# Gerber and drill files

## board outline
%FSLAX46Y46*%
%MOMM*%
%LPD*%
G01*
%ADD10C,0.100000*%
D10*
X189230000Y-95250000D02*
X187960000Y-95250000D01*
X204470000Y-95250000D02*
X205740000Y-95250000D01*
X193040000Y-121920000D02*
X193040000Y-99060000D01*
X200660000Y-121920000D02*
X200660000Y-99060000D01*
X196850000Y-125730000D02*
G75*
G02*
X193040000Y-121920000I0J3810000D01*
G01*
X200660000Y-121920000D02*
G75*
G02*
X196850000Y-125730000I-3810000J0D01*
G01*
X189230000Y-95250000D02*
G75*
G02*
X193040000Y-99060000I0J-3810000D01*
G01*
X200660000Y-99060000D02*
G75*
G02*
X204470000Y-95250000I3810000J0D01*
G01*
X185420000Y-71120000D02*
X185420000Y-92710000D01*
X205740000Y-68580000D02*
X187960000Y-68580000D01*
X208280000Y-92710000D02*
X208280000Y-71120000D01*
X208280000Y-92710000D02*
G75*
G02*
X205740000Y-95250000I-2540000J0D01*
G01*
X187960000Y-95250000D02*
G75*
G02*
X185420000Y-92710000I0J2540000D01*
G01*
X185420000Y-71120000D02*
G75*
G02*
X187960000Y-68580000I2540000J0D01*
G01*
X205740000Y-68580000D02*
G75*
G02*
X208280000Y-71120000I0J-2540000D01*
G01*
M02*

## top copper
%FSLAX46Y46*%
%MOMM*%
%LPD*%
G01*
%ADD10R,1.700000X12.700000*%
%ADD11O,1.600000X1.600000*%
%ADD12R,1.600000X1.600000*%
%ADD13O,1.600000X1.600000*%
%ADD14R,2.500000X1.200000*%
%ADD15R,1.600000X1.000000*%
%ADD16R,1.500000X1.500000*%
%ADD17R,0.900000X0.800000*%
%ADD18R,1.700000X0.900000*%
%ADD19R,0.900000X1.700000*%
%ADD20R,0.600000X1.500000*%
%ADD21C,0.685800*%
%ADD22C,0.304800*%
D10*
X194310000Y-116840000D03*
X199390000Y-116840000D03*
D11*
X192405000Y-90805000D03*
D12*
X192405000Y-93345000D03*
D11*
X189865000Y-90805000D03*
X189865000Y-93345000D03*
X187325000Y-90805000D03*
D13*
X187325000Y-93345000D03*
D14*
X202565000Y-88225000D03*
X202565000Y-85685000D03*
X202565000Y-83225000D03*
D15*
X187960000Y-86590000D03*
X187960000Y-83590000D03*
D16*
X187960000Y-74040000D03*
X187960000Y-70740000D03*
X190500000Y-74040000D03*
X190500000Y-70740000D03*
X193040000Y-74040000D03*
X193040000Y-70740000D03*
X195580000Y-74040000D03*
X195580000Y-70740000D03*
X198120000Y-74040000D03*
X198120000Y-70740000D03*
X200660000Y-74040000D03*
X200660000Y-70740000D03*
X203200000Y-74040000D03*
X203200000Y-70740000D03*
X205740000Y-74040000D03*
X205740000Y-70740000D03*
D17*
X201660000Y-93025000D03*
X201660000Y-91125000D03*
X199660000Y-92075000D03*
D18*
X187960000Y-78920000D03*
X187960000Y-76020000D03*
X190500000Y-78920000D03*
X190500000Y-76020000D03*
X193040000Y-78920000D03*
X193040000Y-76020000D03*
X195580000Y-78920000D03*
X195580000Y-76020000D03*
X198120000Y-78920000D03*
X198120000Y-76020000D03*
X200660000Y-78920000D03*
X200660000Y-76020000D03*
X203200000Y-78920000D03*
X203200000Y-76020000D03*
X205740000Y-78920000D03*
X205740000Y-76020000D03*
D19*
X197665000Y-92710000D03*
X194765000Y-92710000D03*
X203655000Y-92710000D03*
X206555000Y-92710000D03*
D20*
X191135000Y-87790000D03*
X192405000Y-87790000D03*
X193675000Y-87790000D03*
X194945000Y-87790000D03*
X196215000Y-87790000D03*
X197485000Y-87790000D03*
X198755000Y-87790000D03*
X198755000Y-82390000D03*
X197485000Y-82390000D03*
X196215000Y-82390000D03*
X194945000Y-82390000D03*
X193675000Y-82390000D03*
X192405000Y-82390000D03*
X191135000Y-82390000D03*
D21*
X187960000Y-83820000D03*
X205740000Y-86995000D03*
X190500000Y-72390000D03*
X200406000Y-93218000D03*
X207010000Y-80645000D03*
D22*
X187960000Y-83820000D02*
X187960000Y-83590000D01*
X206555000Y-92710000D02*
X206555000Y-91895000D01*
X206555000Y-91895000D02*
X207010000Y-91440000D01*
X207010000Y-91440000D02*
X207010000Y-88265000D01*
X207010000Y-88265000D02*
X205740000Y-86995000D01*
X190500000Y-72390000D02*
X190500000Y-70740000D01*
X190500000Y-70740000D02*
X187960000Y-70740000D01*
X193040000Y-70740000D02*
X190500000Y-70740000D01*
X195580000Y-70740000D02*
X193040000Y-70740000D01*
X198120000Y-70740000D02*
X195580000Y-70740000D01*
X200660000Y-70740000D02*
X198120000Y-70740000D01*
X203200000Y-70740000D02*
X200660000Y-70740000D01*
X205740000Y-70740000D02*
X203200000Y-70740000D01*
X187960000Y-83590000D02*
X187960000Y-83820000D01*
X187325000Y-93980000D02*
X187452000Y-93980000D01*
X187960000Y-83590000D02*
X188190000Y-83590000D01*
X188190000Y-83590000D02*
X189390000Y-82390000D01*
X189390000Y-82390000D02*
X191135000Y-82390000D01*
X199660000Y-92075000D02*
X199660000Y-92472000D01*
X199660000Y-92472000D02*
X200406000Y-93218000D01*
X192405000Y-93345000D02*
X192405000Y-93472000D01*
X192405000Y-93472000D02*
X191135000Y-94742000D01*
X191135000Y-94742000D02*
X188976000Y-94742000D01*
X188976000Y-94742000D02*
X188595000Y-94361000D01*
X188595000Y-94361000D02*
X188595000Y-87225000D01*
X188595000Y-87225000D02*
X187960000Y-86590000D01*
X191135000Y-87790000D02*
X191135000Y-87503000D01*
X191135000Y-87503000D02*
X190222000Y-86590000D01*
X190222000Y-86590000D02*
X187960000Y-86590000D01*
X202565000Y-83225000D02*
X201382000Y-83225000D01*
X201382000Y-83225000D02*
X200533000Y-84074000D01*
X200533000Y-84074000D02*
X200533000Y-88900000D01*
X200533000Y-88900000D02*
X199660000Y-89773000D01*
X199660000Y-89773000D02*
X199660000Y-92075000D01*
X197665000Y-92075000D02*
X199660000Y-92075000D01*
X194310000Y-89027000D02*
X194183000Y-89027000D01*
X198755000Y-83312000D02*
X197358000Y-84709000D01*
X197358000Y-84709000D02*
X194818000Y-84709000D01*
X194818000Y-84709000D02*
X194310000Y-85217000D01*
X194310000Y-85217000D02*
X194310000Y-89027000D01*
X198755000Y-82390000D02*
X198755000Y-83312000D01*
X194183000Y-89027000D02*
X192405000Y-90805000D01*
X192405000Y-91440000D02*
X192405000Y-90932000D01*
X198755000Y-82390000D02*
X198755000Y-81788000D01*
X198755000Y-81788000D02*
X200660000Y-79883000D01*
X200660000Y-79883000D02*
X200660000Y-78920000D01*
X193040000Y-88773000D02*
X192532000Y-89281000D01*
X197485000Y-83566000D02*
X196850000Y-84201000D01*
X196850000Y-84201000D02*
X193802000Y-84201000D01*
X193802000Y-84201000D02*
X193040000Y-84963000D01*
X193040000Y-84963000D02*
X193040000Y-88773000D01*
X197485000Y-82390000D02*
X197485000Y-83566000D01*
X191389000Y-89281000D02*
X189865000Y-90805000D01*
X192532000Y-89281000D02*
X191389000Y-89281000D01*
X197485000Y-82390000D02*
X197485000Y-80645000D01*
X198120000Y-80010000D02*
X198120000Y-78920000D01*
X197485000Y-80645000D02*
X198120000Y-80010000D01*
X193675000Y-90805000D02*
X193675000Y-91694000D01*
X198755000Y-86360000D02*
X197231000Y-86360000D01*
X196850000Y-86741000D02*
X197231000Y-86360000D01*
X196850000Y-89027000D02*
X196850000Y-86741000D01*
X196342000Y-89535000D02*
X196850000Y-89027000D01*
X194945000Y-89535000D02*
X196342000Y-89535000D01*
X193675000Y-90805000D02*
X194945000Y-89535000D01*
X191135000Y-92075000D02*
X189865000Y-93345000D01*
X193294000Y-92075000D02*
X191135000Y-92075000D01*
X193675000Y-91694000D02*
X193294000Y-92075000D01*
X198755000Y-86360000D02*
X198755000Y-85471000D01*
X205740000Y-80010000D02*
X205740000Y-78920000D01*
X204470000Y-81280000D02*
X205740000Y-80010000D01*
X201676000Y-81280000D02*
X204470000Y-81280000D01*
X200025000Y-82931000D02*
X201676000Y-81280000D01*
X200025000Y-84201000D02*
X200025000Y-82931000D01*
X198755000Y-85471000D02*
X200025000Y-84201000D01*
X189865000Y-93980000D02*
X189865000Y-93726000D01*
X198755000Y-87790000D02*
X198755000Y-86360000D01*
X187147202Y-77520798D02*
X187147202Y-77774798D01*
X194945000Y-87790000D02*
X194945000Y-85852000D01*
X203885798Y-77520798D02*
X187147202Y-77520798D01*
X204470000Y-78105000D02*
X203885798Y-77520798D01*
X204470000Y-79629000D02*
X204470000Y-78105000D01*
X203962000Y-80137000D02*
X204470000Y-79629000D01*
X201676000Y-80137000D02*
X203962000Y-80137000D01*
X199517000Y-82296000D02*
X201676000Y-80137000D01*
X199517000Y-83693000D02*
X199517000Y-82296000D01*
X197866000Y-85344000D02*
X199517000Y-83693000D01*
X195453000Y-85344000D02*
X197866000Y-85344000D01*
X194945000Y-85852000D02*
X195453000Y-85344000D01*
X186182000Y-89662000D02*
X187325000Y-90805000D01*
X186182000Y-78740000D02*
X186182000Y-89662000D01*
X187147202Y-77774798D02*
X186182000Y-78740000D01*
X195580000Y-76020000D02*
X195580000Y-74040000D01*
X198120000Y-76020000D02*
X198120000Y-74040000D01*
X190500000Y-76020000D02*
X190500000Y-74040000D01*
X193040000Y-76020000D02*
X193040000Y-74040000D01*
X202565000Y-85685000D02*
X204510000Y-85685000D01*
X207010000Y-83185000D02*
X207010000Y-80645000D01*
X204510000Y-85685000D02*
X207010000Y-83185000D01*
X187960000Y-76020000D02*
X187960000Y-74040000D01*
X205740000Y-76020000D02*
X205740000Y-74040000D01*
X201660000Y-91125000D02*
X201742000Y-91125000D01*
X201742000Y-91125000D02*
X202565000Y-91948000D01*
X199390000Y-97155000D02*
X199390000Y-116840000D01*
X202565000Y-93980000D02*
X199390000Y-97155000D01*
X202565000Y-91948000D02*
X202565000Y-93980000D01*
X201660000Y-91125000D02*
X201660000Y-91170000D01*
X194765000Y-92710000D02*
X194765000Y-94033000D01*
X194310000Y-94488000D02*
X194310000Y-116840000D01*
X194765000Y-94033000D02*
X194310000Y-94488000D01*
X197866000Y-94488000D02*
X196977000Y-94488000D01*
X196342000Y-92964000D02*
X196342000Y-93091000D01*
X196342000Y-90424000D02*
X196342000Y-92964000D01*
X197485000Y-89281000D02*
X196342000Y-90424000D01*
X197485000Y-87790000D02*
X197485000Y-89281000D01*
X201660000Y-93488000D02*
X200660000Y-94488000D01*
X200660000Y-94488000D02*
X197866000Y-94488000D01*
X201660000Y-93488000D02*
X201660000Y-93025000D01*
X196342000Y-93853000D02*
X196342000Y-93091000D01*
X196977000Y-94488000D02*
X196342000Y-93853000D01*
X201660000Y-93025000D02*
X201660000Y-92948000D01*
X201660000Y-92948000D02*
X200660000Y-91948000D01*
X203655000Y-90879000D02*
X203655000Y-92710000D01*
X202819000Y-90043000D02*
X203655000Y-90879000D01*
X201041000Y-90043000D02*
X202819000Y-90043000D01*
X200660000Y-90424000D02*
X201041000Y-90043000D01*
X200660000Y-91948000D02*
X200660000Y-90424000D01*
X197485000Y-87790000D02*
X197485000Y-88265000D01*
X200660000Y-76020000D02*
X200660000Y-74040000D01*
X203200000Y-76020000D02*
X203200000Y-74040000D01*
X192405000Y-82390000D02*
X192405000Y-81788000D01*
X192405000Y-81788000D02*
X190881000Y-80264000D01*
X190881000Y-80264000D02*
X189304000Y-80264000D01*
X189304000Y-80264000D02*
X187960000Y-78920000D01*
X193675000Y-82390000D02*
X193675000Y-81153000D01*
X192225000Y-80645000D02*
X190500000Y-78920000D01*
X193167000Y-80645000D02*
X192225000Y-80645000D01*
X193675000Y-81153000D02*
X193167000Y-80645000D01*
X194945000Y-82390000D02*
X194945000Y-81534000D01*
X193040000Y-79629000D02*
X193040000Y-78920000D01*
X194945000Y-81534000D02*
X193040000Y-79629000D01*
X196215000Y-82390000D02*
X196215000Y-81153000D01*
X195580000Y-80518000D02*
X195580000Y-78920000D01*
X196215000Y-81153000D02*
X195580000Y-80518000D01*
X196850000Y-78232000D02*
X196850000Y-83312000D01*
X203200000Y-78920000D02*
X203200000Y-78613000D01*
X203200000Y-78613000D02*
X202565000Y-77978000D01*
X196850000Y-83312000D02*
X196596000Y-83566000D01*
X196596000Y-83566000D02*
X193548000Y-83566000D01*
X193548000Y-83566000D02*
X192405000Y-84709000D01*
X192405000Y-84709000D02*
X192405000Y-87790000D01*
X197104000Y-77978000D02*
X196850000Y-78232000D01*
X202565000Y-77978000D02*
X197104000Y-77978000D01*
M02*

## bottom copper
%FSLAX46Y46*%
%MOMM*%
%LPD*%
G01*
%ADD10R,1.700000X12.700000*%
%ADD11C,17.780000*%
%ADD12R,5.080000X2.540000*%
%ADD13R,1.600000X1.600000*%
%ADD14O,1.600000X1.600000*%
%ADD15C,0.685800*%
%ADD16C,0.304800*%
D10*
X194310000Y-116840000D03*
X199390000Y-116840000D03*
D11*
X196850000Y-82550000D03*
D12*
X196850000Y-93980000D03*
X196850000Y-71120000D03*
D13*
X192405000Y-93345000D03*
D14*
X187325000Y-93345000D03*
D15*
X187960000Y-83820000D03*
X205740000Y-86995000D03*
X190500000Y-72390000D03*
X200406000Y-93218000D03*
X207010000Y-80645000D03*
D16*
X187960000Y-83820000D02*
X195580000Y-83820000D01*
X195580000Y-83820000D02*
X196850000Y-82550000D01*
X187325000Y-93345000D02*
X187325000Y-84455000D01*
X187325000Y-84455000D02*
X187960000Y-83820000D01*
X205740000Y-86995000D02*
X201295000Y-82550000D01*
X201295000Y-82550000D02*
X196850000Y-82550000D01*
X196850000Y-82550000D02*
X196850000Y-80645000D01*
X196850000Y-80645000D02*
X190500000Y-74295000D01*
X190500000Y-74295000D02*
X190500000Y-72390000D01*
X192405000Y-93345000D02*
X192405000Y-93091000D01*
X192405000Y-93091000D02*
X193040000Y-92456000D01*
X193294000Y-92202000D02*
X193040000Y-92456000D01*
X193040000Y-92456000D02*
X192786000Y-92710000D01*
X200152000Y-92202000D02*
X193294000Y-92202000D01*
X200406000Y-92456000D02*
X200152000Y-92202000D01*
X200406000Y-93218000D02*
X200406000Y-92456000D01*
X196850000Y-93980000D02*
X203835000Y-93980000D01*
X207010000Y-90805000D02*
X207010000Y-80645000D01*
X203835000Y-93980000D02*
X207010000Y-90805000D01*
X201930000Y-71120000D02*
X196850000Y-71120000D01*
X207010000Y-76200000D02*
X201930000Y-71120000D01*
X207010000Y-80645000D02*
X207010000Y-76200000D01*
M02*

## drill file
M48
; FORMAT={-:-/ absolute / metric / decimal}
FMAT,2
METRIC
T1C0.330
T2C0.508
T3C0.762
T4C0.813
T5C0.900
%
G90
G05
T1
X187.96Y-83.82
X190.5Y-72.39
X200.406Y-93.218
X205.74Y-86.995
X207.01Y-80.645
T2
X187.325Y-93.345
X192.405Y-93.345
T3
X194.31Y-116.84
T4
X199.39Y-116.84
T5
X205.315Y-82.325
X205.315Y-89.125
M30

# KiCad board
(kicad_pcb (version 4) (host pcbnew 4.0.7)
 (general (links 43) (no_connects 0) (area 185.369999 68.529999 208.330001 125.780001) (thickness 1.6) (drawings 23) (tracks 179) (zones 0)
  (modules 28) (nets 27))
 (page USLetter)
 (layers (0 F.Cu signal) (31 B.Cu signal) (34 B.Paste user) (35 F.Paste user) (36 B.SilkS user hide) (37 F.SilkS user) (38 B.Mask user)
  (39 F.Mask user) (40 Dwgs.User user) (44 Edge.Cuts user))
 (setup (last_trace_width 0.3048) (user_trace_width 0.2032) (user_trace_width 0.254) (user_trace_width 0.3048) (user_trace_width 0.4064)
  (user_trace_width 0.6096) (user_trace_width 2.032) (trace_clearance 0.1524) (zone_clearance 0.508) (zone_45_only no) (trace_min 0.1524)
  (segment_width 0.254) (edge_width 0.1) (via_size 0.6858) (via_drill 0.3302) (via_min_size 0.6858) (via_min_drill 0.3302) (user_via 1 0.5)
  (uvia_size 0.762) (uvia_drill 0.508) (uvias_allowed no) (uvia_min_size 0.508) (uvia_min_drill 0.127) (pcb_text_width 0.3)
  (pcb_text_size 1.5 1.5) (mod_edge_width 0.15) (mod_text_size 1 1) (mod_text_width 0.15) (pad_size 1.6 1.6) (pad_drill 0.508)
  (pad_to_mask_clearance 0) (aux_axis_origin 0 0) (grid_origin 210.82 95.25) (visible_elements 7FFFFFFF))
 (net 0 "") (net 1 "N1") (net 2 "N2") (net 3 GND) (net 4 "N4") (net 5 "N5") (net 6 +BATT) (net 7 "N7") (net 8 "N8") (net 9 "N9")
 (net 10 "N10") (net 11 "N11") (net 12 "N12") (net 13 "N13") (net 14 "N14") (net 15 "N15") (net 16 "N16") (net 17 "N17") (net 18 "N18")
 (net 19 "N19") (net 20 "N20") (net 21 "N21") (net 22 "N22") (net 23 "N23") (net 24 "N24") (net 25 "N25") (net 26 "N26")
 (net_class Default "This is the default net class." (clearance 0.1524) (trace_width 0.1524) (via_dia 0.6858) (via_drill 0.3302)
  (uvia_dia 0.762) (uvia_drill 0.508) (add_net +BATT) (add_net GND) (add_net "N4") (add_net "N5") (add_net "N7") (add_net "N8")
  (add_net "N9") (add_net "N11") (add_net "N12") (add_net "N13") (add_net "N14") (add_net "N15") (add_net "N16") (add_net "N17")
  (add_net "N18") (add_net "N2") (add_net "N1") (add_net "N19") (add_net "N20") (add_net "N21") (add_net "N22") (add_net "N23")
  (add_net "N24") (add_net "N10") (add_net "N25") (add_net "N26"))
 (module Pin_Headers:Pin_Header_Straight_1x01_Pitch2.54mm (layer F.Cu) (at 194.31 116.84)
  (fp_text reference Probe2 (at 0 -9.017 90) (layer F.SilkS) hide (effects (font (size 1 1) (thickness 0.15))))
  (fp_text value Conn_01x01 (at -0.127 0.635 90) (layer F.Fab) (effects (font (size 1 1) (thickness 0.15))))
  (pad 1 thru_hole rect (at 0 0) (size 1.7 12.7) (drill 0.762) (layers *.Cu *.Mask) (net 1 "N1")))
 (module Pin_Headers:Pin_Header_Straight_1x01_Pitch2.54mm (layer F.Cu) (at 199.39 116.84)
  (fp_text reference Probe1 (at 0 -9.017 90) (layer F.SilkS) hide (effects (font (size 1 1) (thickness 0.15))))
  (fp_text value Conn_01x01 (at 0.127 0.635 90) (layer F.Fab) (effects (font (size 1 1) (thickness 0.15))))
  (pad 1 thru_hole rect (at 0 0) (size 1.7 12.7) (drill 0.8128) (layers *.Cu *.Mask) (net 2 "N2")))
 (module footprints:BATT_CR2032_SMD (layer B.Cu) (at 196.85 82.55 90)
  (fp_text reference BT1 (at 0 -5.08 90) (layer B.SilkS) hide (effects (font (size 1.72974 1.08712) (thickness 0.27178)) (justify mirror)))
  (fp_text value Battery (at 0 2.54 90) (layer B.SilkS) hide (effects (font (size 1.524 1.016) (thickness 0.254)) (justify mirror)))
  (pad 2 smd circle (at 0 0 90) (size 17.78 17.78) (layers B.Cu B.Paste B.Mask) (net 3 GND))
  (pad 1 smd rect (at -11.43 0 90) (size 2.54 5.08) (layers B.Cu B.Paste B.Mask) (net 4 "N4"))
  (pad 1 smd rect (at 11.43 0 90) (size 2.54 5.08) (layers B.Cu B.Paste B.Mask) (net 4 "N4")))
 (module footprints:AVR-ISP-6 (layer F.Cu) (at 192.405 90.805 270)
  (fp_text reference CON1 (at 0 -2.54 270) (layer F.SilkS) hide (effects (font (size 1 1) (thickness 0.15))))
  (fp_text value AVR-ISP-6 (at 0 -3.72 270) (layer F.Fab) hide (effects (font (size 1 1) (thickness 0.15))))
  (pad 1 smd oval (at 0 0 270) (size 1.6 1.6) (layers F.Cu F.Paste F.Mask) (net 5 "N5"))
  (pad 2 thru_hole rect (at 2.54 0 270) (size 1.6 1.6) (drill 0.508) (layers *.Cu *.Mask) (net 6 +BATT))
  (pad 3 smd oval (at 0 2.54 270) (size 1.6 1.6) (layers F.Cu F.Paste F.Mask) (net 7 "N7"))
  (pad 4 smd oval (at 2.54 2.54 270) (size 1.6 1.6) (layers F.Cu F.Paste F.Mask) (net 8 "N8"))
  (pad 5 smd oval (at 0 5.08 270) (size 1.6 1.6) (layers F.Cu F.Paste F.Mask) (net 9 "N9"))
  (pad 6 thru_hole oval (at 2.54 5.08 270) (size 1.6 1.6) (drill 0.508) (layers *.Cu *.Mask) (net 3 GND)))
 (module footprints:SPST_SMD (layer F.Cu) (at 202.565 85.725 90)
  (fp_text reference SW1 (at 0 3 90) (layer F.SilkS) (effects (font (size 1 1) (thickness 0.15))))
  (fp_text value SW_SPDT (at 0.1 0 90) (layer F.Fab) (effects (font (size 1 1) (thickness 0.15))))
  (pad "" np_thru_hole circle (at 3.4 2.75 90) (size 0.9 0.9) (drill 0.9) (layers *.Cu *.Mask))
  (pad 1 smd rect (at -2.5 0 90) (size 1.2 2.5) (layers F.Cu F.Paste F.Mask) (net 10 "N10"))
  (pad 2 smd rect (at 0.04 0 90) (size 1.2 2.5) (layers F.Cu F.Paste F.Mask) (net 4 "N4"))
  (pad 3 smd rect (at 2.5 0 90) (size 1.2 2.5) (layers F.Cu F.Paste F.Mask) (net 6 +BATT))
  (pad "" np_thru_hole circle (at -3.4 2.75 90) (size 0.9 0.9) (drill 0.9) (layers *.Cu *.Mask)))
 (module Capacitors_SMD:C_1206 (layer F.Cu) (at 187.96 85.09 90)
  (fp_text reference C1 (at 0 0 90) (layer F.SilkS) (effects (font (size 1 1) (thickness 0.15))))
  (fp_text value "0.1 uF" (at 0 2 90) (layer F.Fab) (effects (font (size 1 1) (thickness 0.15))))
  (pad 1 smd rect (at -1.5 0 90) (size 1 1.6) (layers F.Cu F.Paste F.Mask) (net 6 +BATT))
  (pad 2 smd rect (at 1.5 0 90) (size 1 1.6) (layers F.Cu F.Paste F.Mask) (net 3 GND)))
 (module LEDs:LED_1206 (layer F.Cu) (at 187.96 72.39 270)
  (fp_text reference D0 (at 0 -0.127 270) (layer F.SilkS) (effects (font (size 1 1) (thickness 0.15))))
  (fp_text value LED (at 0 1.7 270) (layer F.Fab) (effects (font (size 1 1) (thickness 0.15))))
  (pad 2 smd rect (at 1.65 0 90) (size 1.5 1.5) (layers F.Cu F.Paste F.Mask) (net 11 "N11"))
  (pad 1 smd rect (at -1.65 0 90) (size 1.5 1.5) (layers F.Cu F.Paste F.Mask) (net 3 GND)))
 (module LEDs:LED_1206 (layer F.Cu) (at 190.5 72.39 270)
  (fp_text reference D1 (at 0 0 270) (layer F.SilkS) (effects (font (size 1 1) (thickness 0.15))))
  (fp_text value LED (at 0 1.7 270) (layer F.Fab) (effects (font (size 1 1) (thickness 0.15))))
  (pad 2 smd rect (at 1.65 0 90) (size 1.5 1.5) (layers F.Cu F.Paste F.Mask) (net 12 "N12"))
  (pad 1 smd rect (at -1.65 0 90) (size 1.5 1.5) (layers F.Cu F.Paste F.Mask) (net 3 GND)))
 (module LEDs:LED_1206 (layer F.Cu) (at 193.04 72.39 270)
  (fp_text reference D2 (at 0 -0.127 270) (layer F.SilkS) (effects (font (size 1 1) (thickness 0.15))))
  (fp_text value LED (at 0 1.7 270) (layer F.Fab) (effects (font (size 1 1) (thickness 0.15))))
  (pad 2 smd rect (at 1.65 0 90) (size 1.5 1.5) (layers F.Cu F.Paste F.Mask) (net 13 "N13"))
  (pad 1 smd rect (at -1.65 0 90) (size 1.5 1.5) (layers F.Cu F.Paste F.Mask) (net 3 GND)))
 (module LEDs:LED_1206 (layer F.Cu) (at 195.58 72.39 270)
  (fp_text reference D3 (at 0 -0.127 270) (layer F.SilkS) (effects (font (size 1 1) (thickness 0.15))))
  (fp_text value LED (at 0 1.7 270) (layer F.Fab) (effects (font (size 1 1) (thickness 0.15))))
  (pad 2 smd rect (at 1.65 0 90) (size 1.5 1.5) (layers F.Cu F.Paste F.Mask) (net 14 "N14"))
  (pad 1 smd rect (at -1.65 0 90) (size 1.5 1.5) (layers F.Cu F.Paste F.Mask) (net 3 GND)))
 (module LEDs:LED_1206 (layer F.Cu) (at 198.12 72.39 270)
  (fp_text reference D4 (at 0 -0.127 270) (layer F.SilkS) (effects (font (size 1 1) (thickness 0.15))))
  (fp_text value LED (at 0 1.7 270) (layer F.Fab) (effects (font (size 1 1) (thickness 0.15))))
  (pad 2 smd rect (at 1.65 0 90) (size 1.5 1.5) (layers F.Cu F.Paste F.Mask) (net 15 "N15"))
  (pad 1 smd rect (at -1.65 0 90) (size 1.5 1.5) (layers F.Cu F.Paste F.Mask) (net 3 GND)))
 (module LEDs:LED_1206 (layer F.Cu) (at 200.66 72.39 270)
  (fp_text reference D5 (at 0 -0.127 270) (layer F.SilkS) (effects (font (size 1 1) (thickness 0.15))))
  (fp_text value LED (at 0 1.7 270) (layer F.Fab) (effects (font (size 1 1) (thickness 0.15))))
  (pad 2 smd rect (at 1.65 0 90) (size 1.5 1.5) (layers F.Cu F.Paste F.Mask) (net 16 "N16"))
  (pad 1 smd rect (at -1.65 0 90) (size 1.5 1.5) (layers F.Cu F.Paste F.Mask) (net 3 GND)))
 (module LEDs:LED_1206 (layer F.Cu) (at 203.2 72.39 270)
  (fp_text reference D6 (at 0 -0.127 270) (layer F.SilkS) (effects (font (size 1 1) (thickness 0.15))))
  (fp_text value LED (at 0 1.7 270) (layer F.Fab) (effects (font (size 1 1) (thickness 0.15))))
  (pad 2 smd rect (at 1.65 0 90) (size 1.5 1.5) (layers F.Cu F.Paste F.Mask) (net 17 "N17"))
  (pad 1 smd rect (at -1.65 0 90) (size 1.5 1.5) (layers F.Cu F.Paste F.Mask) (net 3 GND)))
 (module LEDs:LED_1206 (layer F.Cu) (at 205.74 72.39 270)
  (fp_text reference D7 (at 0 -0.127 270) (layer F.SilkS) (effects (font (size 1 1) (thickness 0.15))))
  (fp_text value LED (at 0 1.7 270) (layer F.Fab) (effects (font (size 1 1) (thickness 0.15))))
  (pad 2 smd rect (at 1.65 0 90) (size 1.5 1.5) (layers F.Cu F.Paste F.Mask) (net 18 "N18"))
  (pad 1 smd rect (at -1.65 0 90) (size 1.5 1.5) (layers F.Cu F.Paste F.Mask) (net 3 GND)))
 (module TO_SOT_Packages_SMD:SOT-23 (layer F.Cu) (at 200.66 92.075 180)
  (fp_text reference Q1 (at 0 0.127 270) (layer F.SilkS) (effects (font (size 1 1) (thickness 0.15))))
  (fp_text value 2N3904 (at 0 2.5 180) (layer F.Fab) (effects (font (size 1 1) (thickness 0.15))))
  (pad 1 smd rect (at -1 -0.95 180) (size 0.9 0.8) (layers F.Cu F.Paste F.Mask) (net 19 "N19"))
  (pad 2 smd rect (at -1 0.95 180) (size 0.9 0.8) (layers F.Cu F.Paste F.Mask) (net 2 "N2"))
  (pad 3 smd rect (at 1 0 180) (size 0.9 0.8) (layers F.Cu F.Paste F.Mask) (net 6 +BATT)))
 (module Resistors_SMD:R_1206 (layer F.Cu) (at 187.96 77.47 90)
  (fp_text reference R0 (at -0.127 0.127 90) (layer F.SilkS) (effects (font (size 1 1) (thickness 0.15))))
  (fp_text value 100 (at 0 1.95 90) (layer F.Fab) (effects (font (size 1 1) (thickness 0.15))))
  (pad 1 smd rect (at -1.45 0 90) (size 0.9 1.7) (layers F.Cu F.Paste F.Mask) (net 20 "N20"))
  (pad 2 smd rect (at 1.45 0 90) (size 0.9 1.7) (layers F.Cu F.Paste F.Mask) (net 11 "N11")))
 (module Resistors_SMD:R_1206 (layer F.Cu) (at 190.5 77.47 90)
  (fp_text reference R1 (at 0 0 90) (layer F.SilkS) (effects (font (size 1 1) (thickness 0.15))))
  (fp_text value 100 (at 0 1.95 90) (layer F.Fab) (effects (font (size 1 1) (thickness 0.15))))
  (pad 1 smd rect (at -1.45 0 90) (size 0.9 1.7) (layers F.Cu F.Paste F.Mask) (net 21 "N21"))
  (pad 2 smd rect (at 1.45 0 90) (size 0.9 1.7) (layers F.Cu F.Paste F.Mask) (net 12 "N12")))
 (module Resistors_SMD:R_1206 (layer F.Cu) (at 193.04 77.47 90)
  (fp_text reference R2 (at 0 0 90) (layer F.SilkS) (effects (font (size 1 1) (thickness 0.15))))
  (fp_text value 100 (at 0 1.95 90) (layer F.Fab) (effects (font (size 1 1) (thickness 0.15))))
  (pad 1 smd rect (at -1.45 0 90) (size 0.9 1.7) (layers F.Cu F.Paste F.Mask) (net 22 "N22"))
  (pad 2 smd rect (at 1.45 0 90) (size 0.9 1.7) (layers F.Cu F.Paste F.Mask) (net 13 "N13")))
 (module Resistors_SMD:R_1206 (layer F.Cu) (at 195.58 77.47 90)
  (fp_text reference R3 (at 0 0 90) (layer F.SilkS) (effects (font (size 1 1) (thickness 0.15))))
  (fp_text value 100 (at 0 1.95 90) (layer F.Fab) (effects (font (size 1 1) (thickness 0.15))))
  (pad 1 smd rect (at -1.45 0 90) (size 0.9 1.7) (layers F.Cu F.Paste F.Mask) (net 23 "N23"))
  (pad 2 smd rect (at 1.45 0 90) (size 0.9 1.7) (layers F.Cu F.Paste F.Mask) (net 14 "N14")))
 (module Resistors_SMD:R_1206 (layer F.Cu) (at 198.12 77.47 90)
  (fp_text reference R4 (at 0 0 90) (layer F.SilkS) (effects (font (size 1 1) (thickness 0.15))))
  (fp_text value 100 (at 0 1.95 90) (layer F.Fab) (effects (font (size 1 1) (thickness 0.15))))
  (pad 1 smd rect (at -1.45 0 90) (size 0.9 1.7) (layers F.Cu F.Paste F.Mask) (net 7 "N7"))
  (pad 2 smd rect (at 1.45 0 90) (size 0.9 1.7) (layers F.Cu F.Paste F.Mask) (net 15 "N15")))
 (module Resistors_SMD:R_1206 (layer F.Cu) (at 200.66 77.47 90)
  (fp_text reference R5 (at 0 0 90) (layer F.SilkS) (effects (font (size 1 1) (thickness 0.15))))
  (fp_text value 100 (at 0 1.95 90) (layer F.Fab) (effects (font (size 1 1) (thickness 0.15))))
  (pad 1 smd rect (at -1.45 0 90) (size 0.9 1.7) (layers F.Cu F.Paste F.Mask) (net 5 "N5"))
  (pad 2 smd rect (at 1.45 0 90) (size 0.9 1.7) (layers F.Cu F.Paste F.Mask) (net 16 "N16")))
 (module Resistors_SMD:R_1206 (layer F.Cu) (at 203.2 77.47 90)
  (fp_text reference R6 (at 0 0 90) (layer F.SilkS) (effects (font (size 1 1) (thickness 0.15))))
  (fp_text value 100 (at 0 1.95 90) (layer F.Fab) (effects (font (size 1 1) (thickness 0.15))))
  (pad 1 smd rect (at -1.45 0 90) (size 0.9 1.7) (layers F.Cu F.Paste F.Mask) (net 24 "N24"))
  (pad 2 smd rect (at 1.45 0 90) (size 0.9 1.7) (layers F.Cu F.Paste F.Mask) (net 17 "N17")))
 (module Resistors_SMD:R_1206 (layer F.Cu) (at 205.74 77.47 90)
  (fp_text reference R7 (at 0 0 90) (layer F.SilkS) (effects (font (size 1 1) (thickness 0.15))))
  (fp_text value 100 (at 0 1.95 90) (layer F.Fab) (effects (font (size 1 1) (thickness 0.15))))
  (pad 1 smd rect (at -1.45 0 90) (size 0.9 1.7) (layers F.Cu F.Paste F.Mask) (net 8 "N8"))
  (pad 2 smd rect (at 1.45 0 90) (size 0.9 1.7) (layers F.Cu F.Paste F.Mask) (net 18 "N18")))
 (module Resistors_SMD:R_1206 (layer F.Cu) (at 196.215 92.71 180)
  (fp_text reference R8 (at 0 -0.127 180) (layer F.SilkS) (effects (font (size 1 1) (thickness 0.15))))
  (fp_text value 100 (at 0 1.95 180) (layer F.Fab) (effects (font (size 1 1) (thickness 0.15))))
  (pad 1 smd rect (at -1.45 0 180) (size 0.9 1.7) (layers F.Cu F.Paste F.Mask) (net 6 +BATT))
  (pad 2 smd rect (at 1.45 0 180) (size 0.9 1.7) (layers F.Cu F.Paste F.Mask) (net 1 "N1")))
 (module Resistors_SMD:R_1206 (layer F.Cu) (at 205.105 92.71)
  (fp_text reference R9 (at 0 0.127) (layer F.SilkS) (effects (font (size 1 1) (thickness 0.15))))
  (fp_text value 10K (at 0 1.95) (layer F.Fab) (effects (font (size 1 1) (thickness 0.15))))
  (pad 1 smd rect (at -1.45 0) (size 0.9 1.7) (layers F.Cu F.Paste F.Mask) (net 19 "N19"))
  (pad 2 smd rect (at 1.45 0) (size 0.9 1.7) (layers F.Cu F.Paste F.Mask) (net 3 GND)))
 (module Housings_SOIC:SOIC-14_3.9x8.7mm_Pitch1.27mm (layer F.Cu) (at 194.945 85.09 90)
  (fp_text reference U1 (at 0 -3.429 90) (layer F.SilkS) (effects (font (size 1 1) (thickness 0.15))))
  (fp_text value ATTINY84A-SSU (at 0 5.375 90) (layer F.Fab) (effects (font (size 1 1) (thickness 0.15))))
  (pad 1 smd rect (at -2.7 -3.81 90) (size 1.5 0.6) (layers F.Cu F.Paste F.Mask) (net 6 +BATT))
  (pad 2 smd rect (at -2.7 -2.54 90) (size 1.5 0.6) (layers F.Cu F.Paste F.Mask) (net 24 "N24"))
  (pad 3 smd rect (at -2.7 -1.27 90) (size 1.5 0.6) (layers F.Cu F.Paste F.Mask) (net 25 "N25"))
  (pad 4 smd rect (at -2.7 0 90) (size 1.5 0.6) (layers F.Cu F.Paste F.Mask) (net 9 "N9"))
  (pad 5 smd rect (at -2.7 1.27 90) (size 1.5 0.6) (layers F.Cu F.Paste F.Mask) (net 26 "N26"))
  (pad 6 smd rect (at -2.7 2.54 90) (size 1.5 0.6) (layers F.Cu F.Paste F.Mask) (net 19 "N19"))
  (pad 7 smd rect (at -2.7 3.81 90) (size 1.5 0.6) (layers F.Cu F.Paste F.Mask) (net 8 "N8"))
  (pad 8 smd rect (at 2.7 3.81 90) (size 1.5 0.6) (layers F.Cu F.Paste F.Mask) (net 5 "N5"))
  (pad 9 smd rect (at 2.7 2.54 90) (size 1.5 0.6) (layers F.Cu F.Paste F.Mask) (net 7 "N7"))
  (pad 10 smd rect (at 2.7 1.27 90) (size 1.5 0.6) (layers F.Cu F.Paste F.Mask) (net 23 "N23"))
  (pad 11 smd rect (at 2.7 0 90) (size 1.5 0.6) (layers F.Cu F.Paste F.Mask) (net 22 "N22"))
  (pad 12 smd rect (at 2.7 -1.27 90) (size 1.5 0.6) (layers F.Cu F.Paste F.Mask) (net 21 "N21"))
  (pad 13 smd rect (at 2.7 -2.54 90) (size 1.5 0.6) (layers F.Cu F.Paste F.Mask) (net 20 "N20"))
  (pad 14 smd rect (at 2.7 -3.81 90) (size 1.5 0.6) (layers F.Cu F.Paste F.Mask) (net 3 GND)))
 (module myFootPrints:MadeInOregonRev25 (layer F.Cu) (at 196.977 99.695 270)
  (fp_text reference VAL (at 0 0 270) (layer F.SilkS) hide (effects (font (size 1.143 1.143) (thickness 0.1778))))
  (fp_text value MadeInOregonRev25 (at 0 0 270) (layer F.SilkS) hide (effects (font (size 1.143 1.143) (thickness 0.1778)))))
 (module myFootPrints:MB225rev (layer F.Cu) (at 196.85 106.68 270)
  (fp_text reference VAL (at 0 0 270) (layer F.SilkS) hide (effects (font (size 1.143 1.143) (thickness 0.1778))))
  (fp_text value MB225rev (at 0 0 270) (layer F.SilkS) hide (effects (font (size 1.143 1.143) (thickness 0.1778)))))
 (gr_line (start 189.23 95.25) (end 187.96 95.25) (angle 90) (layer Edge.Cuts) (width 0.1))
 (gr_line (start 204.47 95.25) (end 205.74 95.25) (angle 90) (layer Edge.Cuts) (width 0.1))
 (gr_line (start 193.04 121.92) (end 193.04 99.06) (angle 90) (layer Edge.Cuts) (width 0.1))
 (gr_line (start 200.66 121.92) (end 200.66 99.06) (angle 90) (layer Edge.Cuts) (width 0.1))
 (gr_arc (start 196.85 121.92) (end 196.85 125.73) (angle 90) (layer Edge.Cuts) (width 0.1))
 (gr_arc (start 196.85 121.92) (end 200.66 121.92) (angle 90) (layer Edge.Cuts) (width 0.1))
 (gr_arc (start 189.23 99.06) (end 189.23 95.25) (angle 90) (layer Edge.Cuts) (width 0.1))
 (gr_arc (start 204.47 99.06) (end 200.66 99.06) (angle 90) (layer Edge.Cuts) (width 0.1))
 (gr_line (start 185.42 71.12) (end 185.42 92.71) (angle 90) (layer Edge.Cuts) (width 0.1))
 (gr_line (start 205.74 68.58) (end 187.96 68.58) (angle 90) (layer Edge.Cuts) (width 0.1))
 (gr_line (start 208.28 92.71) (end 208.28 71.12) (angle 90) (layer Edge.Cuts) (width 0.1))
 (gr_arc (start 205.74 92.71) (end 208.28 92.71) (angle 90) (layer Edge.Cuts) (width 0.1))
 (gr_arc (start 187.96 92.71) (end 187.96 95.25) (angle 90) (layer Edge.Cuts) (width 0.1))
 (gr_arc (start 187.96 71.12) (end 185.42 71.12) (angle 90) (layer Edge.Cuts) (width 0.1))
 (gr_arc (start 205.74 71.12) (end 205.74 68.58) (angle 90) (layer Edge.Cuts) (width 0.1))
 (segment (start 187.96 83.82) (end 195.58 83.82) (width 0.3048) (layer B.Cu) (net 3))
 (segment (start 195.58 83.82) (end 196.85 82.55) (width 0.3048) (layer B.Cu) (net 3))
 (segment (start 187.325 93.345) (end 187.325 84.455) (width 0.3048) (layer B.Cu) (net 3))
 (via (at 187.96 83.82) (size 0.6858) (drill 0.3302) (layers F.Cu B.Cu) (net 3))
 (segment (start 187.325 84.455) (end 187.96 83.82) (width 0.3048) (layer B.Cu) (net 3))
 (segment (start 187.96 83.82) (end 187.96 83.59) (width 0.3048) (layer F.Cu) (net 3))
 (segment (start 206.555 92.71) (end 206.555 91.895) (width 0.3048) (layer F.Cu) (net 3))
 (segment (start 206.555 91.895) (end 207.01 91.44) (width 0.3048) (layer F.Cu) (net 3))
 (segment (start 207.01 91.44) (end 207.01 88.265) (width 0.3048) (layer F.Cu) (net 3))
 (segment (start 207.01 88.265) (end 205.74 86.995) (width 0.3048) (layer F.Cu) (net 3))
 (via (at 205.74 86.995) (size 0.6858) (drill 0.3302) (layers F.Cu B.Cu) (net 3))
 (segment (start 205.74 86.995) (end 201.295 82.55) (width 0.3048) (layer B.Cu) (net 3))
 (segment (start 201.295 82.55) (end 196.85 82.55) (width 0.3048) (layer B.Cu) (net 3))
 (segment (start 196.85 82.55) (end 196.85 80.645) (width 0.3048) (layer B.Cu) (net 3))
 (segment (start 196.85 80.645) (end 190.5 74.295) (width 0.3048) (layer B.Cu) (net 3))
 (segment (start 190.5 74.295) (end 190.5 72.39) (width 0.3048) (layer B.Cu) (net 3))
 (via (at 190.5 72.39) (size 0.6858) (drill 0.3302) (layers F.Cu B.Cu) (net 3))
 (segment (start 190.5 72.39) (end 190.5 70.74) (width 0.3048) (layer F.Cu) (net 3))
 (segment (start 190.5 70.74) (end 187.96 70.74) (width 0.3048) (layer F.Cu) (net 3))
 (segment (start 193.04 70.74) (end 190.5 70.74) (width 0.3048) (layer F.Cu) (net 3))
 (segment (start 195.58 70.74) (end 193.04 70.74) (width 0.3048) (layer F.Cu) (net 3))
 (segment (start 198.12 70.74) (end 195.58 70.74) (width 0.3048) (layer F.Cu) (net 3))
 (segment (start 200.66 70.74) (end 198.12 70.74) (width 0.3048) (layer F.Cu) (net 3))
 (segment (start 203.2 70.74) (end 200.66 70.74) (width 0.3048) (layer F.Cu) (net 3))
 (segment (start 205.74 70.74) (end 203.2 70.74) (width 0.3048) (layer F.Cu) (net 3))
 (segment (start 187.96 83.59) (end 187.96 83.82) (width 0.3048) (layer F.Cu) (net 3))
 (segment (start 187.325 93.98) (end 187.452 93.98) (width 0.3048) (layer F.Cu) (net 3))
 (segment (start 187.96 83.59) (end 188.19 83.59) (width 0.3048) (layer F.Cu) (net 3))
 (segment (start 188.19 83.59) (end 189.39 82.39) (width 0.3048) (layer F.Cu) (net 3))
 (segment (start 189.39 82.39) (end 191.135 82.39) (width 0.3048) (layer F.Cu) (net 3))
 (segment (start 192.405 93.345) (end 192.405 93.091) (width 0.3048) (layer B.Cu) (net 6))
 (segment (start 192.405 93.091) (end 193.04 92.456) (width 0.3048) (layer B.Cu) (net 6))
 (segment (start 199.66 92.075) (end 199.66 92.472) (width 0.3048) (layer F.Cu) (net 6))
 (segment (start 199.66 92.472) (end 200.406 93.218) (width 0.3048) (layer F.Cu) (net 6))
 (segment (start 193.294 92.202) (end 193.04 92.456) (width 0.3048) (layer B.Cu) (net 6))
 (segment (start 193.04 92.456) (end 192.786 92.71) (width 0.3048) (layer B.Cu) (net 6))
 (segment (start 200.152 92.202) (end 193.294 92.202) (width 0.3048) (layer B.Cu) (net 6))
 (segment (start 200.406 92.456) (end 200.152 92.202) (width 0.3048) (layer B.Cu) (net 6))
 (segment (start 200.406 93.218) (end 200.406 92.456) (width 0.3048) (layer B.Cu) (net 6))
 (via (at 200.406 93.218) (size 0.6858) (drill 0.3302) (layers F.Cu B.Cu) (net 6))
 (segment (start 192.405 93.345) (end 192.405 93.472) (width 0.3048) (layer F.Cu) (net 6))
 (segment (start 192.405 93.472) (end 191.135 94.742) (width 0.3048) (layer F.Cu) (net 6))
 (segment (start 191.135 94.742) (end 188.976 94.742) (width 0.3048) (layer F.Cu) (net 6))
 (segment (start 188.976 94.742) (end 188.595 94.361) (width 0.3048) (layer F.Cu) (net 6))
 (segment (start 188.595 94.361) (end 188.595 87.225) (width 0.3048) (layer F.Cu) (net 6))
 (segment (start 188.595 87.225) (end 187.96 86.59) (width 0.3048) (layer F.Cu) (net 6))
 (segment (start 191.135 87.79) (end 191.135 87.503) (width 0.3048) (layer F.Cu) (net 6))
 (segment (start 191.135 87.503) (end 190.222 86.59) (width 0.3048) (layer F.Cu) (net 6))
 (segment (start 190.222 86.59) (end 187.96 86.59) (width 0.3048) (layer F.Cu) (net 6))
 (segment (start 202.565 83.225) (end 201.382 83.225) (width 0.3048) (layer F.Cu) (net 6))
 (segment (start 201.382 83.225) (end 200.533 84.074) (width 0.3048) (layer F.Cu) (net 6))
 (segment (start 200.533 84.074) (end 200.533 88.9) (width 0.3048) (layer F.Cu) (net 6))
 (segment (start 200.533 88.9) (end 199.66 89.773) (width 0.3048) (layer F.Cu) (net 6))
 (segment (start 199.66 89.773) (end 199.66 92.075) (width 0.3048) (layer F.Cu) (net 6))
 (segment (start 197.665 92.075) (end 199.66 92.075) (width 0.3048) (layer F.Cu) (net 6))
 (segment (start 194.31 89.027) (end 194.183 89.027) (width 0.3048) (layer F.Cu) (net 5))
 (segment (start 198.755 83.312) (end 197.358 84.709) (width 0.3048) (layer F.Cu) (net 5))
 (segment (start 197.358 84.709) (end 194.818 84.709) (width 0.3048) (layer F.Cu) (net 5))
 (segment (start 194.818 84.709) (end 194.31 85.217) (width 0.3048) (layer F.Cu) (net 5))
 (segment (start 194.31 85.217) (end 194.31 89.027) (width 0.3048) (layer F.Cu) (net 5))
 (segment (start 198.755 82.39) (end 198.755 83.312) (width 0.3048) (layer F.Cu) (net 5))
 (segment (start 194.183 89.027) (end 192.405 90.805) (width 0.3048) (layer F.Cu) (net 5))
 (segment (start 192.405 91.44) (end 192.405 90.932) (width 0.3048) (layer F.Cu) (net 5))
 (segment (start 198.755 82.39) (end 198.755 81.788) (width 0.3048) (layer F.Cu) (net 5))
 (segment (start 198.755 81.788) (end 200.66 79.883) (width 0.3048) (layer F.Cu) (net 5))
 (segment (start 200.66 79.883) (end 200.66 78.92) (width 0.3048) (layer F.Cu) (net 5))
 (segment (start 193.04 88.773) (end 192.532 89.281) (width 0.3048) (layer F.Cu) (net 7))
 (segment (start 197.485 83.566) (end 196.85 84.201) (width 0.3048) (layer F.Cu) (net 7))
 (segment (start 196.85 84.201) (end 193.802 84.201) (width 0.3048) (layer F.Cu) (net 7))
 (segment (start 193.802 84.201) (end 193.04 84.963) (width 0.3048) (layer F.Cu) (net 7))
 (segment (start 193.04 84.963) (end 193.04 88.773) (width 0.3048) (layer F.Cu) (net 7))
 (segment (start 197.485 82.39) (end 197.485 83.566) (width 0.3048) (layer F.Cu) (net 7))
 (segment (start 191.389 89.281) (end 189.865 90.805) (width 0.3048) (layer F.Cu) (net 7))
 (segment (start 192.532 89.281) (end 191.389 89.281) (width 0.3048) (layer F.Cu) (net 7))
 (segment (start 197.485 82.39) (end 197.485 80.645) (width 0.3048) (layer F.Cu) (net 7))
 (segment (start 198.12 80.01) (end 198.12 78.92) (width 0.3048) (layer F.Cu) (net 7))
 (segment (start 197.485 80.645) (end 198.12 80.01) (width 0.3048) (layer F.Cu) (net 7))
 (segment (start 193.675 90.805) (end 193.675 91.694) (width 0.3048) (layer F.Cu) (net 8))
 (segment (start 198.755 86.36) (end 197.231 86.36) (width 0.3048) (layer F.Cu) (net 8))
 (segment (start 196.85 86.741) (end 197.231 86.36) (width 0.3048) (layer F.Cu) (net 8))
 (segment (start 196.85 89.027) (end 196.85 86.741) (width 0.3048) (layer F.Cu) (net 8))
 (segment (start 196.342 89.535) (end 196.85 89.027) (width 0.3048) (layer F.Cu) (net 8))
 (segment (start 194.945 89.535) (end 196.342 89.535) (width 0.3048) (layer F.Cu) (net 8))
 (segment (start 193.675 90.805) (end 194.945 89.535) (width 0.3048) (layer F.Cu) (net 8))
 (segment (start 191.135 92.075) (end 189.865 93.345) (width 0.3048) (layer F.Cu) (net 8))
 (segment (start 193.294 92.075) (end 191.135 92.075) (width 0.3048) (layer F.Cu) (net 8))
 (segment (start 193.675 91.694) (end 193.294 92.075) (width 0.3048) (layer F.Cu) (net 8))
 (segment (start 198.755 86.36) (end 198.755 85.471) (width 0.3048) (layer F.Cu) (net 8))
 (segment (start 205.74 80.01) (end 205.74 78.92) (width 0.3048) (layer F.Cu) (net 8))
 (segment (start 204.47 81.28) (end 205.74 80.01) (width 0.3048) (layer F.Cu) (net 8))
 (segment (start 201.676 81.28) (end 204.47 81.28) (width 0.3048) (layer F.Cu) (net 8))
 (segment (start 200.025 82.931) (end 201.676 81.28) (width 0.3048) (layer F.Cu) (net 8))
 (segment (start 200.025 84.201) (end 200.025 82.931) (width 0.3048) (layer F.Cu) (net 8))
 (segment (start 198.755 85.471) (end 200.025 84.201) (width 0.3048) (layer F.Cu) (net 8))
 (segment (start 189.865 93.98) (end 189.865 93.726) (width 0.3048) (layer F.Cu) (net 8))
 (segment (start 198.755 87.79) (end 198.755 86.36) (width 0.3048) (layer F.Cu) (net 8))
 (segment (start 187.147202 77.520798) (end 187.147202 77.774798) (width 0.3048) (layer F.Cu) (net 9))
 (segment (start 194.945 87.79) (end 194.945 85.852) (width 0.3048) (layer F.Cu) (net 9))
 (segment (start 203.885798 77.520798) (end 187.147202 77.520798) (width 0.3048) (layer F.Cu) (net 9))
 (segment (start 204.47 78.105) (end 203.885798 77.520798) (width 0.3048) (layer F.Cu) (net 9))
 (segment (start 204.47 79.629) (end 204.47 78.105) (width 0.3048) (layer F.Cu) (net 9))
 (segment (start 203.962 80.137) (end 204.47 79.629) (width 0.3048) (layer F.Cu) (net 9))
 (segment (start 201.676 80.137) (end 203.962 80.137) (width 0.3048) (layer F.Cu) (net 9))
 (segment (start 199.517 82.296) (end 201.676 80.137) (width 0.3048) (layer F.Cu) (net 9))
 (segment (start 199.517 83.693) (end 199.517 82.296) (width 0.3048) (layer F.Cu) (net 9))
 (segment (start 197.866 85.344) (end 199.517 83.693) (width 0.3048) (layer F.Cu) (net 9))
 (segment (start 195.453 85.344) (end 197.866 85.344) (width 0.3048) (layer F.Cu) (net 9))
 (segment (start 194.945 85.852) (end 195.453 85.344) (width 0.3048) (layer F.Cu) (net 9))
 (segment (start 186.182 89.662) (end 187.325 90.805) (width 0.3048) (layer F.Cu) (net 9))
 (segment (start 186.182 78.74) (end 186.182 89.662) (width 0.3048) (layer F.Cu) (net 9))
 (segment (start 187.147202 77.774798) (end 186.182 78.74) (width 0.3048) (layer F.Cu) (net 9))
 (segment (start 195.58 76.02) (end 195.58 74.04) (width 0.3048) (layer F.Cu) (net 14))
 (segment (start 198.12 76.02) (end 198.12 74.04) (width 0.3048) (layer F.Cu) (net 15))
 (segment (start 190.5 76.02) (end 190.5 74.04) (width 0.3048) (layer F.Cu) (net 12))
 (segment (start 193.04 76.02) (end 193.04 74.04) (width 0.3048) (layer F.Cu) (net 13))
 (segment (start 196.85 93.98) (end 203.835 93.98) (width 0.3048) (layer B.Cu) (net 4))
 (segment (start 207.01 90.805) (end 207.01 80.645) (width 0.3048) (layer B.Cu) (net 4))
 (segment (start 203.835 93.98) (end 207.01 90.805) (width 0.3048) (layer B.Cu) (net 4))
 (segment (start 202.565 85.685) (end 204.51 85.685) (width 0.3048) (layer F.Cu) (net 4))
 (segment (start 201.93 71.12) (end 196.85 71.12) (width 0.3048) (layer B.Cu) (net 4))
 (segment (start 207.01 76.2) (end 201.93 71.12) (width 0.3048) (layer B.Cu) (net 4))
 (segment (start 207.01 80.645) (end 207.01 76.2) (width 0.3048) (layer B.Cu) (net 4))
 (via (at 207.01 80.645) (size 0.6858) (drill 0.3302) (layers F.Cu B.Cu) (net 4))
 (segment (start 207.01 83.185) (end 207.01 80.645) (width 0.3048) (layer F.Cu) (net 4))
 (segment (start 204.51 85.685) (end 207.01 83.185) (width 0.3048) (layer F.Cu) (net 4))
 (segment (start 187.96 76.02) (end 187.96 74.04) (width 0.3048) (layer F.Cu) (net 11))
 (segment (start 205.74 76.02) (end 205.74 74.04) (width 0.3048) (layer F.Cu) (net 18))
 (segment (start 201.66 91.125) (end 201.742 91.125) (width 0.3048) (layer F.Cu) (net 2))
 (segment (start 201.742 91.125) (end 202.565 91.948) (width 0.3048) (layer F.Cu) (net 2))
 (segment (start 199.39 97.155) (end 199.39 116.84) (width 0.3048) (layer F.Cu) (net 2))
 (segment (start 202.565 93.98) (end 199.39 97.155) (width 0.3048) (layer F.Cu) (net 2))
 (segment (start 202.565 91.948) (end 202.565 93.98) (width 0.3048) (layer F.Cu) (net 2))
 (segment (start 201.66 91.125) (end 201.66 91.17) (width 0.3048) (layer F.Cu) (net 2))
 (segment (start 194.765 92.71) (end 194.765 94.033) (width 0.3048) (layer F.Cu) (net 1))
 (segment (start 194.31 94.488) (end 194.31 116.84) (width 0.3048) (layer F.Cu) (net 1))
 (segment (start 194.765 94.033) (end 194.31 94.488) (width 0.3048) (layer F.Cu) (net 1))
 (segment (start 197.866 94.488) (end 196.977 94.488) (width 0.3048) (layer F.Cu) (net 19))
 (segment (start 196.342 92.964) (end 196.342 93.091) (width 0.3048) (layer F.Cu) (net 19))
 (segment (start 196.342 90.424) (end 196.342 92.964) (width 0.3048) (layer F.Cu) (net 19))
 (segment (start 197.485 89.281) (end 196.342 90.424) (width 0.3048) (layer F.Cu) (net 19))
 (segment (start 197.485 87.79) (end 197.485 89.281) (width 0.3048) (layer F.Cu) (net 19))
 (segment (start 201.66 93.488) (end 200.66 94.488) (width 0.3048) (layer F.Cu) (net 19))
 (segment (start 200.66 94.488) (end 197.866 94.488) (width 0.3048) (layer F.Cu) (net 19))
 (segment (start 201.66 93.488) (end 201.66 93.025) (width 0.3048) (layer F.Cu) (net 19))
 (segment (start 196.342 93.853) (end 196.342 93.091) (width 0.3048) (layer F.Cu) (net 19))
 (segment (start 196.977 94.488) (end 196.342 93.853) (width 0.3048) (layer F.Cu) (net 19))
 (segment (start 201.66 93.025) (end 201.66 92.948) (width 0.3048) (layer F.Cu) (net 19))
 (segment (start 201.66 92.948) (end 200.66 91.948) (width 0.3048) (layer F.Cu) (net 19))
 (segment (start 203.655 90.879) (end 203.655 92.71) (width 0.3048) (layer F.Cu) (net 19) (status 20))
 (segment (start 202.819 90.043) (end 203.655 90.879) (width 0.3048) (layer F.Cu) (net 19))
 (segment (start 201.041 90.043) (end 202.819 90.043) (width 0.3048) (layer F.Cu) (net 19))
 (segment (start 200.66 90.424) (end 201.041 90.043) (width 0.3048) (layer F.Cu) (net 19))
 (segment (start 200.66 91.948) (end 200.66 90.424) (width 0.3048) (layer F.Cu) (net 19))
 (segment (start 197.485 87.79) (end 197.485 88.265) (width 0.3048) (layer F.Cu) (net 19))
 (segment (start 200.66 76.02) (end 200.66 74.04) (width 0.3048) (layer F.Cu) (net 16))
 (segment (start 203.2 76.02) (end 203.2 74.04) (width 0.3048) (layer F.Cu) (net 17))
 (segment (start 192.405 82.39) (end 192.405 81.788) (width 0.3048) (layer F.Cu) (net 20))
 (segment (start 192.405 81.788) (end 190.881 80.264) (width 0.3048) (layer F.Cu) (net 20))
 (segment (start 190.881 80.264) (end 189.304 80.264) (width 0.3048) (layer F.Cu) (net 20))
 (segment (start 189.304 80.264) (end 187.96 78.92) (width 0.3048) (layer F.Cu) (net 20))
 (segment (start 193.675 82.39) (end 193.675 81.153) (width 0.3048) (layer F.Cu) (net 21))
 (segment (start 192.225 80.645) (end 190.5 78.92) (width 0.3048) (layer F.Cu) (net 21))
 (segment (start 193.167 80.645) (end 192.225 80.645) (width 0.3048) (layer F.Cu) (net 21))
 (segment (start 193.675 81.153) (end 193.167 80.645) (width 0.3048) (layer F.Cu) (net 21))
 (segment (start 194.945 82.39) (end 194.945 81.534) (width 0.3048) (layer F.Cu) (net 22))
 (segment (start 193.04 79.629) (end 193.04 78.92) (width 0.3048) (layer F.Cu) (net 22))
 (segment (start 194.945 81.534) (end 193.04 79.629) (width 0.3048) (layer F.Cu) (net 22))
 (segment (start 196.215 82.39) (end 196.215 81.153) (width 0.3048) (layer F.Cu) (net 23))
 (segment (start 195.58 80.518) (end 195.58 78.92) (width 0.3048) (layer F.Cu) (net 23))
 (segment (start 196.215 81.153) (end 195.58 80.518) (width 0.3048) (layer F.Cu) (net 23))
 (segment (start 196.85 78.232) (end 196.85 83.312) (width 0.3048) (layer F.Cu) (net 24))
 (segment (start 203.2 78.92) (end 203.2 78.613) (width 0.3048) (layer F.Cu) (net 24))
 (segment (start 203.2 78.613) (end 202.565 77.978) (width 0.3048) (layer F.Cu) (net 24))
 (segment (start 196.85 83.312) (end 196.596 83.566) (width 0.3048) (layer F.Cu) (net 24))
 (segment (start 196.596 83.566) (end 193.548 83.566) (width 0.3048) (layer F.Cu) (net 24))
 (segment (start 193.548 83.566) (end 192.405 84.709) (width 0.3048) (layer F.Cu) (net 24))
 (segment (start 192.405 84.709) (end 192.405 87.79) (width 0.3048) (layer F.Cu) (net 24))
 (segment (start 197.104 77.978) (end 196.85 78.232) (width 0.3048) (layer F.Cu) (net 24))
 (segment (start 202.565 77.978) (end 197.104 77.978) (width 0.3048) (layer F.Cu) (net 24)))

